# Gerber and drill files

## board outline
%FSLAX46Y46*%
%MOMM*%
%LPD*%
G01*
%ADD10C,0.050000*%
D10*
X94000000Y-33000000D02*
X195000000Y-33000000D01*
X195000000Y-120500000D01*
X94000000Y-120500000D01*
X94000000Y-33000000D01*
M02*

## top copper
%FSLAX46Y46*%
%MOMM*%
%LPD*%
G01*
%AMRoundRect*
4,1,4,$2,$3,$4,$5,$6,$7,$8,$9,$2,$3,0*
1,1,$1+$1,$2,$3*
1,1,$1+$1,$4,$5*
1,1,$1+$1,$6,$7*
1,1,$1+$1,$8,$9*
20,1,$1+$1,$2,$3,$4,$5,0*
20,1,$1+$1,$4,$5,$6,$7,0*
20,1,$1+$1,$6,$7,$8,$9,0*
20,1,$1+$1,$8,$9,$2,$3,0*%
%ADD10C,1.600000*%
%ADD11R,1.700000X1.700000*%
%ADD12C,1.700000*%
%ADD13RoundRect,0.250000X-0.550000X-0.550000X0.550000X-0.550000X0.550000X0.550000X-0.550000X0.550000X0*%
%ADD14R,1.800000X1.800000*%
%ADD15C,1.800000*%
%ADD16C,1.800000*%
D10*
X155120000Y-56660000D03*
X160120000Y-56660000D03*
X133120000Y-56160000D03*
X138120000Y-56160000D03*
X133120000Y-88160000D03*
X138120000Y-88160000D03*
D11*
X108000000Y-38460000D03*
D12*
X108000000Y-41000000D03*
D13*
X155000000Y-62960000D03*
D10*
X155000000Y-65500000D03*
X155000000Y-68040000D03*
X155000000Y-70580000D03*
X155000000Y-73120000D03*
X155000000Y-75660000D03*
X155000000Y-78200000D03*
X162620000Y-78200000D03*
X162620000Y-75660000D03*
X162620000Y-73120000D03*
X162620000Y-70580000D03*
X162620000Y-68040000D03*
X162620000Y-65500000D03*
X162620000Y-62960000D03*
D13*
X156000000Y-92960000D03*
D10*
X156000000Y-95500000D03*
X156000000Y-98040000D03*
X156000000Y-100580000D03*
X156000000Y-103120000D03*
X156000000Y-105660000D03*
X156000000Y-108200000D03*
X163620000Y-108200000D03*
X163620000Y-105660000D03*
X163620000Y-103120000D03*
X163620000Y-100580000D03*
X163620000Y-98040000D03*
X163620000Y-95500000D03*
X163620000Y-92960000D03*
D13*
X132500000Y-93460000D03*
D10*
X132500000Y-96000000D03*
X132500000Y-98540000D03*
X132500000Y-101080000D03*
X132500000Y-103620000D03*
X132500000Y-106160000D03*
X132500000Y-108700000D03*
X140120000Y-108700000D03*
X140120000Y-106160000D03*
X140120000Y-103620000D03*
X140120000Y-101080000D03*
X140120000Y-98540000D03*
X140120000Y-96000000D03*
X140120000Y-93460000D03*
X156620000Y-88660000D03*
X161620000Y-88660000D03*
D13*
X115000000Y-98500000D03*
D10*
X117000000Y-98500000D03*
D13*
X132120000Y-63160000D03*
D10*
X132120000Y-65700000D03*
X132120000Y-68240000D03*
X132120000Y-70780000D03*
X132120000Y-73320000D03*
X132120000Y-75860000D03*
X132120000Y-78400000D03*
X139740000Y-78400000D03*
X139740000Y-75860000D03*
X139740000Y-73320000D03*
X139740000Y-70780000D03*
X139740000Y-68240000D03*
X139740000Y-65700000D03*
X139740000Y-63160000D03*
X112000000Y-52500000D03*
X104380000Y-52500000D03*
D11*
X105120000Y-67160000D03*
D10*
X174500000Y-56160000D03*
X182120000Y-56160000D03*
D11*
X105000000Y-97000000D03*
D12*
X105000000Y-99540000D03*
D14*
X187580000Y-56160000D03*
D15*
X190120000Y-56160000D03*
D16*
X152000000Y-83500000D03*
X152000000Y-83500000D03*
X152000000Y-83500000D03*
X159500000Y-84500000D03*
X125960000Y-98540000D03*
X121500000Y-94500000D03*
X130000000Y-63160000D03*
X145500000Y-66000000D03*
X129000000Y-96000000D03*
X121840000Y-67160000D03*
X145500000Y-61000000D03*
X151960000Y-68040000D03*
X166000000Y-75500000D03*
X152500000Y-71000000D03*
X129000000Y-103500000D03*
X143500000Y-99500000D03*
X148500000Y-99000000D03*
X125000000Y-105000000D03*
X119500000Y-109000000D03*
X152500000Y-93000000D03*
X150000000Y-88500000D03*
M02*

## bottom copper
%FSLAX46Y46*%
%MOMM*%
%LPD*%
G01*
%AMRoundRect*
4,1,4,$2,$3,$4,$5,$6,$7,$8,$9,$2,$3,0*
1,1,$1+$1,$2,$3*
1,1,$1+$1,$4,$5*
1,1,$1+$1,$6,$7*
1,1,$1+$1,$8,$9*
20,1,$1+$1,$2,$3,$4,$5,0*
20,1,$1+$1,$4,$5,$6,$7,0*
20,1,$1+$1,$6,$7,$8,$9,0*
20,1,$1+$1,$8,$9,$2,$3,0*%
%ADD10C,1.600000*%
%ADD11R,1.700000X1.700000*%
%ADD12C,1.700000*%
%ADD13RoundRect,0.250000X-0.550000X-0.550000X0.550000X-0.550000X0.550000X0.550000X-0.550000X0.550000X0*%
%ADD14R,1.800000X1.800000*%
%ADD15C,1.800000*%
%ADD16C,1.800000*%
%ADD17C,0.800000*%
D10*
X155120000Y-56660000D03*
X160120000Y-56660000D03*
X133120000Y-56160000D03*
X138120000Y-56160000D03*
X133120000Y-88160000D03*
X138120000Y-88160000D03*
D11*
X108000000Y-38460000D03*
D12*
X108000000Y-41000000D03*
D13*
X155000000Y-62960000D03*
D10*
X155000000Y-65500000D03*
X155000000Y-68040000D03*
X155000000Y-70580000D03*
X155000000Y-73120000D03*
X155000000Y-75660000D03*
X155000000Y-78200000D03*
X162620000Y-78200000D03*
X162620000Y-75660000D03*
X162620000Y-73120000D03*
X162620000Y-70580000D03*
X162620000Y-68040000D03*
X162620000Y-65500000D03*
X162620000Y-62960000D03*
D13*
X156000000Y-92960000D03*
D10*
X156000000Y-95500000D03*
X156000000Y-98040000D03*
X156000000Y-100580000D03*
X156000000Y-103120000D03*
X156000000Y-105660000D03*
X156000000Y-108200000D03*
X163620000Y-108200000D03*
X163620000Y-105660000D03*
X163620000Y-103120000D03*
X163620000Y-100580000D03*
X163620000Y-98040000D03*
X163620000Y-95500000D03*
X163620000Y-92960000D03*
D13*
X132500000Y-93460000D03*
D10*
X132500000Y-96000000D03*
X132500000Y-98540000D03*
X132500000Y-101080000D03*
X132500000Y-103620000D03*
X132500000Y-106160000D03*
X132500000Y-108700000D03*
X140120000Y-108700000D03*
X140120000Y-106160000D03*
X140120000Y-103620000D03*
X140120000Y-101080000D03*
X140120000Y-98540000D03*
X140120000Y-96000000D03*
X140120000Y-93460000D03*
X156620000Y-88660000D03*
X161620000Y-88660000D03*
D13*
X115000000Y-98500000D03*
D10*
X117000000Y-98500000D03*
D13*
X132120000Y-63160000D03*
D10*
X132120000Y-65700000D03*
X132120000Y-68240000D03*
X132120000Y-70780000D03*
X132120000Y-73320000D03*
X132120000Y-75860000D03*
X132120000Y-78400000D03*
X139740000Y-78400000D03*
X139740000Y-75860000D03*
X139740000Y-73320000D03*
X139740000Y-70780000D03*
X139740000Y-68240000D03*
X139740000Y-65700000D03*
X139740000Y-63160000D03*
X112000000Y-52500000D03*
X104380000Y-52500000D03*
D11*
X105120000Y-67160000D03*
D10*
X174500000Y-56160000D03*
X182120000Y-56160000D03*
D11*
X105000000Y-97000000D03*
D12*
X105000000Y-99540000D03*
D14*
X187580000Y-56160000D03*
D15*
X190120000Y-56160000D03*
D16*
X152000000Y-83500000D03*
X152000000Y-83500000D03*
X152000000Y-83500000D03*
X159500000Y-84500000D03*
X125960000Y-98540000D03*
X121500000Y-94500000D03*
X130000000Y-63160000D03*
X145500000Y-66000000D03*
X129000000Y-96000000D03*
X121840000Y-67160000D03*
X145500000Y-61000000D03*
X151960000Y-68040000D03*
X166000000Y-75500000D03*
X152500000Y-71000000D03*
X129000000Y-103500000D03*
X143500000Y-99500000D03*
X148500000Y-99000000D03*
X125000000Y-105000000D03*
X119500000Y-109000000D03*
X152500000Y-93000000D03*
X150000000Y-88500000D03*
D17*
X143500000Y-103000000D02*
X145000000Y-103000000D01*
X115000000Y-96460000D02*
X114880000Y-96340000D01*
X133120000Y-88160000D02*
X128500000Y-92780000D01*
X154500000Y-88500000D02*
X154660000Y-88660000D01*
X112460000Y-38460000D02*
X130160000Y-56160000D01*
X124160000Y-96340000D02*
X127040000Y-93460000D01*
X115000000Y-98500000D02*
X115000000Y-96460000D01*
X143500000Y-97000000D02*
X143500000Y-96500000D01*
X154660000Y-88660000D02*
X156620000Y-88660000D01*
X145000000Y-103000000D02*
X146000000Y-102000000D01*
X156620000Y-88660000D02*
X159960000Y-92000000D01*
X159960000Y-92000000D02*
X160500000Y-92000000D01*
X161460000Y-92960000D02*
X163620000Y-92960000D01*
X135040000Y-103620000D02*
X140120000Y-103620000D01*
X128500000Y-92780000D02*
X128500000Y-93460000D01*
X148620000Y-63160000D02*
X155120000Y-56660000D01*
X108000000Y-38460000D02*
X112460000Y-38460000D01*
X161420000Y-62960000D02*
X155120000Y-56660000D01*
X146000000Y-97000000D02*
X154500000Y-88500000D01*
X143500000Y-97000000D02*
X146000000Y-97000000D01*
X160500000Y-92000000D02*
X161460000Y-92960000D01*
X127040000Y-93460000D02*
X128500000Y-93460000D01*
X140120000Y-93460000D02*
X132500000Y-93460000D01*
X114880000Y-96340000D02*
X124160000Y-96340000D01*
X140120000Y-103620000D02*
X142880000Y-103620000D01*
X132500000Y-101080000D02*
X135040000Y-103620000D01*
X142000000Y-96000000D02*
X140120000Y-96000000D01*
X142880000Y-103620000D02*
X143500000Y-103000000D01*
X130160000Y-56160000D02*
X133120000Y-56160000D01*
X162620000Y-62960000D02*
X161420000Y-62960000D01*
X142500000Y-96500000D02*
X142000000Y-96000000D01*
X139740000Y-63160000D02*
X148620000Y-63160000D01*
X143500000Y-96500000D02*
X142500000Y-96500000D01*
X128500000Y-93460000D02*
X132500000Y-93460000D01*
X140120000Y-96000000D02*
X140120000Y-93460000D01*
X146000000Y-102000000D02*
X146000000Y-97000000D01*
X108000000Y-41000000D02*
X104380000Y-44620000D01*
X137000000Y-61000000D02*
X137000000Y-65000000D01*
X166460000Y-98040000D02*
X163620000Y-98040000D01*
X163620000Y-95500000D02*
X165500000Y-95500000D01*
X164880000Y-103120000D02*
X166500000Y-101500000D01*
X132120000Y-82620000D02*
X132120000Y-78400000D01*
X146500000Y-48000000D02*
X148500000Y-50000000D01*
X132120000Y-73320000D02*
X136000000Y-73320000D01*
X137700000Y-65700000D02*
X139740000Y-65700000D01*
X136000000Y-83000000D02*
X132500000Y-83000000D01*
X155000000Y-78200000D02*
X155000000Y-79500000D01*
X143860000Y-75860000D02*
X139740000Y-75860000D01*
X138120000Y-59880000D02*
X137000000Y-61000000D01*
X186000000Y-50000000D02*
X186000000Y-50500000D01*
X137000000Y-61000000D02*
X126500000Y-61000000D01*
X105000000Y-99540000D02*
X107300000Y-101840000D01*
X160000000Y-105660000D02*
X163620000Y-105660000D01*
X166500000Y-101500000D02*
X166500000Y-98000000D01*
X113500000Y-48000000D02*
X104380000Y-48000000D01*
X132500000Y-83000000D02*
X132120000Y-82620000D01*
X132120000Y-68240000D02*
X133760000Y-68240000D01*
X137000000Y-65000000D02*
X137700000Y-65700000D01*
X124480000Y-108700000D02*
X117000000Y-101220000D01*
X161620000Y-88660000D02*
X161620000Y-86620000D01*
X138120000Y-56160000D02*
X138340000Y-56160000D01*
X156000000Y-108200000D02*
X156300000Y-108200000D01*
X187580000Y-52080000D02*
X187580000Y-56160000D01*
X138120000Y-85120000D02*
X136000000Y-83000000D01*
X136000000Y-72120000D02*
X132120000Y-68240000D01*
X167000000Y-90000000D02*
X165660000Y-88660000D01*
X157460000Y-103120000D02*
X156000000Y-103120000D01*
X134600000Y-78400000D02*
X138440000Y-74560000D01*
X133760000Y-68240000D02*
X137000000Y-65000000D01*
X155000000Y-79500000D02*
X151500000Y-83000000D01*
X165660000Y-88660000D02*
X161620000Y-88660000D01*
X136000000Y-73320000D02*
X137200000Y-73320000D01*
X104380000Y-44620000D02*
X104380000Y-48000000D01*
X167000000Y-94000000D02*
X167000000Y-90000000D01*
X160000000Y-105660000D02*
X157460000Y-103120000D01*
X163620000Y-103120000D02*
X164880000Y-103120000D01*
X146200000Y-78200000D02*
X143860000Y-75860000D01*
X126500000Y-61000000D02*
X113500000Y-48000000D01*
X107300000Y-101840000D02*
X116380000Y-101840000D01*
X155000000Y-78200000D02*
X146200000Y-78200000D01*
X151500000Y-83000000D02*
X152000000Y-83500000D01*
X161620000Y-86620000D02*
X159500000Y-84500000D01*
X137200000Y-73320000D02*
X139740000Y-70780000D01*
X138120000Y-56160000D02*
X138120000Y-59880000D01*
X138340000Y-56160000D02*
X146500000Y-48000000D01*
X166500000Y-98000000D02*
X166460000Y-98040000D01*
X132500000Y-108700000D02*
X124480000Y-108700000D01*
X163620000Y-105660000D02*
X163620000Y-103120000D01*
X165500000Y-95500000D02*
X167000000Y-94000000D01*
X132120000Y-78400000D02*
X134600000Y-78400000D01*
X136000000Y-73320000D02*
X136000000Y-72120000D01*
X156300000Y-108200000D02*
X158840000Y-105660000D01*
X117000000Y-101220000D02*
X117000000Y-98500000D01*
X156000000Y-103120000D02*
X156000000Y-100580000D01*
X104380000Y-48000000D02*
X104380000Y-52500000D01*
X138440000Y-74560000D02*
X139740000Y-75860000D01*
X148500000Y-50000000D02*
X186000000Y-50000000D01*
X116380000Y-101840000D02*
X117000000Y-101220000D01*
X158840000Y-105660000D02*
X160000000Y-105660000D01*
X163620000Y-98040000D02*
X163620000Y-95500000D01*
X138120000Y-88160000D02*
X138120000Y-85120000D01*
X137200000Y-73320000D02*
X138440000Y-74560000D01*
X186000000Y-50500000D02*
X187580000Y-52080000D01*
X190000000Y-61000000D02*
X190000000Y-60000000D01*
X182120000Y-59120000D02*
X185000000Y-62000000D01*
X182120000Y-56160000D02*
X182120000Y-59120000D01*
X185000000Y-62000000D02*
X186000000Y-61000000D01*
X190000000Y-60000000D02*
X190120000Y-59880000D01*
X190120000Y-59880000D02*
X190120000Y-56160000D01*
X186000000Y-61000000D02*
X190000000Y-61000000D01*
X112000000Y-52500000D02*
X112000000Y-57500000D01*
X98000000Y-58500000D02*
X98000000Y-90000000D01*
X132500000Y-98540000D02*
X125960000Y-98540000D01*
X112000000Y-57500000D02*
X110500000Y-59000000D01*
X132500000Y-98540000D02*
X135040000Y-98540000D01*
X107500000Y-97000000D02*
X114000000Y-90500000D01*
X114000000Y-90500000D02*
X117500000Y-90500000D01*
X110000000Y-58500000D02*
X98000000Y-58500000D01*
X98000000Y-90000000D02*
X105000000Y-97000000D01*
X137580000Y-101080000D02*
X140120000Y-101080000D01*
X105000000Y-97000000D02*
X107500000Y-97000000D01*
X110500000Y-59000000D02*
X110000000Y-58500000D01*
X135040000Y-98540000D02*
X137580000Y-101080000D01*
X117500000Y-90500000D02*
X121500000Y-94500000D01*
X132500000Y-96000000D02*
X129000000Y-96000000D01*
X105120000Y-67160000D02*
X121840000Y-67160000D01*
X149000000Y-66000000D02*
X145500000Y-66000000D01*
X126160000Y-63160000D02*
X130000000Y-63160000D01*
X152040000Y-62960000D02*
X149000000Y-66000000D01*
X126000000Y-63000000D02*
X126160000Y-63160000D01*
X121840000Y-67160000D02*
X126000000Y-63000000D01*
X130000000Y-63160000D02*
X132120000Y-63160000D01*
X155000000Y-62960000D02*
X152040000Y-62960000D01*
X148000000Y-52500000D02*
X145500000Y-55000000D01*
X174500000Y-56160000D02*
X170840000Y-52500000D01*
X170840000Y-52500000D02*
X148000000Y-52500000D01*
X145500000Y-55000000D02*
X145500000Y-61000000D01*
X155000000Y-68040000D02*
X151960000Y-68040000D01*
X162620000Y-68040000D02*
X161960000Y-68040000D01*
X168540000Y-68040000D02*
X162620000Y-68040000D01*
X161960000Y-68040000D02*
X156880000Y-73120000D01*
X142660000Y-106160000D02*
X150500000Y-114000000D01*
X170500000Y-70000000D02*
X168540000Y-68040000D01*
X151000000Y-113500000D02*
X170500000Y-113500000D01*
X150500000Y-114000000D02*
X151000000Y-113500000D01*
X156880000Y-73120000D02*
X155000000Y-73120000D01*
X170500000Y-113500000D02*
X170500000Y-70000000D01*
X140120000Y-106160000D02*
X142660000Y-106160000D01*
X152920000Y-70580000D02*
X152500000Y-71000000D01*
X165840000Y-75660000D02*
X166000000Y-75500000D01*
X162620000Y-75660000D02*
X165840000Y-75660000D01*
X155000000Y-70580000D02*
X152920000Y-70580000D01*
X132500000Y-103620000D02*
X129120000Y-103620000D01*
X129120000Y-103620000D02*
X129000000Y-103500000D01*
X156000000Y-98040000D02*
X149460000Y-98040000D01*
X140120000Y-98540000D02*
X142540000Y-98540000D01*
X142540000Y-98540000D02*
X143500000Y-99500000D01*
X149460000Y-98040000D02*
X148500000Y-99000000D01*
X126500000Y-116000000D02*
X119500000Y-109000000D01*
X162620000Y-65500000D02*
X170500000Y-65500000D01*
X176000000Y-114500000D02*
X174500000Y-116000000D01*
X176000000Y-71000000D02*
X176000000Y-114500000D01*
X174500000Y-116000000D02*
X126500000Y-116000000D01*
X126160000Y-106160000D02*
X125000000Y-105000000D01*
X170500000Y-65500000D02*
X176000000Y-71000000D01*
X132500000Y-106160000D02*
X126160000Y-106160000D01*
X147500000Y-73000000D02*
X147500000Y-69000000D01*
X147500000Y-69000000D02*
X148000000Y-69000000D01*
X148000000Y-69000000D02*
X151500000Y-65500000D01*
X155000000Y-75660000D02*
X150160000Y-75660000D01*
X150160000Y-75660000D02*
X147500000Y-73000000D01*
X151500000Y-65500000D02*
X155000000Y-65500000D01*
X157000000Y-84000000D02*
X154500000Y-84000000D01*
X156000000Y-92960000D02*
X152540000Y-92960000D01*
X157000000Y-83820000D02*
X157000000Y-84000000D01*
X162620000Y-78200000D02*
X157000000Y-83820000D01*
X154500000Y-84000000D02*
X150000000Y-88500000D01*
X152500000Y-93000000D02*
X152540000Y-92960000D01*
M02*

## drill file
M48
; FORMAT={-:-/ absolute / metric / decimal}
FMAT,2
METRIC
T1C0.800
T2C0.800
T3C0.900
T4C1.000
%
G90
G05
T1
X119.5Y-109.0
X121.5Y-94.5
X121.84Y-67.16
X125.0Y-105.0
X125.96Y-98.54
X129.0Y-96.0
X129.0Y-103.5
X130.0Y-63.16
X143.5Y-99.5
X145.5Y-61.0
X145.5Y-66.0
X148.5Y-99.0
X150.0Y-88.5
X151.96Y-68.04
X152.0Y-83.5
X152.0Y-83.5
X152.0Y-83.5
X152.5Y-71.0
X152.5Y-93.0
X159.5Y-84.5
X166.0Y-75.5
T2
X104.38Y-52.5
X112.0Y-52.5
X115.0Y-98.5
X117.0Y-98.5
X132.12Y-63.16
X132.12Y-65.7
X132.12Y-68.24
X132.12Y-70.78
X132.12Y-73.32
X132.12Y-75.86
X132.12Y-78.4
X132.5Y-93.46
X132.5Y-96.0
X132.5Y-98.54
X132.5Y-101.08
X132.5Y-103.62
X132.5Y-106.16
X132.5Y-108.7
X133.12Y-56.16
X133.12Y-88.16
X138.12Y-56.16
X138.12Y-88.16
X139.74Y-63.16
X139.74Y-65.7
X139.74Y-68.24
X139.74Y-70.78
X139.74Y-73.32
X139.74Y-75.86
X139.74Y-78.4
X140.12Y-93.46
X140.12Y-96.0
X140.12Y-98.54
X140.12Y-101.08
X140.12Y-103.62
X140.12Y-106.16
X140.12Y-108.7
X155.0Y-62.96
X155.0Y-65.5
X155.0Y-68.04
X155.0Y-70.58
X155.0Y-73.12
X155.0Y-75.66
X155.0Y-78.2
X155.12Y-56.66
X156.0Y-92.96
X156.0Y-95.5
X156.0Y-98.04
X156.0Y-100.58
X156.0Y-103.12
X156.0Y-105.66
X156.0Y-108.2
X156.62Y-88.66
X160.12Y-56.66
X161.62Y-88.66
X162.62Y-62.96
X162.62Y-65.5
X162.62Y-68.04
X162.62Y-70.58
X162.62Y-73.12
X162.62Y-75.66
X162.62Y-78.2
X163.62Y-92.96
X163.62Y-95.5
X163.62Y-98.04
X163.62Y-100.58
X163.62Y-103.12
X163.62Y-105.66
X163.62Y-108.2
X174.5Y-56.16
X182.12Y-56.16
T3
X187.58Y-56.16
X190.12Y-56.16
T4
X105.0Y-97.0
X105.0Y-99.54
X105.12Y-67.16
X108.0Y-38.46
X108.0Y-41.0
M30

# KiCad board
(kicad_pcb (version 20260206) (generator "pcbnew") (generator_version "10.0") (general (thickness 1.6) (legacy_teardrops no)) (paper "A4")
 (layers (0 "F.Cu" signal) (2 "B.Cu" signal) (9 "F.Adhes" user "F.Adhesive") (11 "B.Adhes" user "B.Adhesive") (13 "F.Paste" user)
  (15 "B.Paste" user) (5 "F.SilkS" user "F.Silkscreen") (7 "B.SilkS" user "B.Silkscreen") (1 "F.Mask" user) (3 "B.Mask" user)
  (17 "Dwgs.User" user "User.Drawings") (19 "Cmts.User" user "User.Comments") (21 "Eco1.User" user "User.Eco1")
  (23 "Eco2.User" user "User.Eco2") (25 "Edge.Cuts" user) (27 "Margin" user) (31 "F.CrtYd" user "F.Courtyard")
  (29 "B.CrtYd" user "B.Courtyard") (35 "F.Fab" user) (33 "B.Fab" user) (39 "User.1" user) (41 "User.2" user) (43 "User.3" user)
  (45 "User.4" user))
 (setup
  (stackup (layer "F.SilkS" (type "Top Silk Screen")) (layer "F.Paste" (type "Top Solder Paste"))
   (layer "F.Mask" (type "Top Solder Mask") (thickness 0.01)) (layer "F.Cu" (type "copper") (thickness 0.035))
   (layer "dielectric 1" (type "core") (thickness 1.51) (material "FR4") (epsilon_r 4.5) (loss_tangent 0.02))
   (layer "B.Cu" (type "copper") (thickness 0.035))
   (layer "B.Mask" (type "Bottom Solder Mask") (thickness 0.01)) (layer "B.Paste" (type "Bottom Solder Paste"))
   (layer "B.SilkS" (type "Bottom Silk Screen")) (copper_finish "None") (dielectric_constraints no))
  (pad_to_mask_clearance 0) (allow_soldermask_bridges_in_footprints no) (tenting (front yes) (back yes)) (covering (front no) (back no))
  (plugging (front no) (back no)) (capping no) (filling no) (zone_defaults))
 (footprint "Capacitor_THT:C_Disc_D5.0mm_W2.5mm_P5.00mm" (layer "F.Cu") (at 155.12 56.66)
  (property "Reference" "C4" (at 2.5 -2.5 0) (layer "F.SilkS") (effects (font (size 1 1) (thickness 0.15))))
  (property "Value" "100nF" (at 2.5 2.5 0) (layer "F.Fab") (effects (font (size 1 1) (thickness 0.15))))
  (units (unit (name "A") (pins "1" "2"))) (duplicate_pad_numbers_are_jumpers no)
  (pad "1" thru_hole circle (at 0 0) (size 1.6 1.6) (drill 0.8) (layers "*.Cu" "*.Mask") (remove_unused_layers no) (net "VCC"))
  (pad "2" thru_hole circle (at 5 0) (size 1.6 1.6) (drill 0.8) (layers "*.Cu" "*.Mask") (remove_unused_layers no) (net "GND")))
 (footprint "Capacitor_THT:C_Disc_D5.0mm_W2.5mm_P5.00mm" (layer "F.Cu") (at 133.12 56.16)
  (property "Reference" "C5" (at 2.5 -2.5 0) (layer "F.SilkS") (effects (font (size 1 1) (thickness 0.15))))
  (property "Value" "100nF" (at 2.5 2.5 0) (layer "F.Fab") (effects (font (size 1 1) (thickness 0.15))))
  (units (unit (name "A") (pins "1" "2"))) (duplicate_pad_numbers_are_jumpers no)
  (pad "1" thru_hole circle (at 0 0) (size 1.6 1.6) (drill 0.8) (layers "*.Cu" "*.Mask") (remove_unused_layers no) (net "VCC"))
  (pad "2" thru_hole circle (at 5 0) (size 1.6 1.6) (drill 0.8) (layers "*.Cu" "*.Mask") (remove_unused_layers no) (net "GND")))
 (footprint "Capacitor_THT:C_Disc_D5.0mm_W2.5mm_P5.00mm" (layer "F.Cu") (at 133.12 88.16)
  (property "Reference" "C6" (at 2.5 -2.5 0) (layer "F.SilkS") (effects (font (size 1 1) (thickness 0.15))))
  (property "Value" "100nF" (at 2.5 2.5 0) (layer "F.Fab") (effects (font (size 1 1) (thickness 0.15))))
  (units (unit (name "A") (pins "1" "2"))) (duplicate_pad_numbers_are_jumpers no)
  (pad "1" thru_hole circle (at 0 0) (size 1.6 1.6) (drill 0.8) (layers "*.Cu" "*.Mask") (remove_unused_layers no) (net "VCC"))
  (pad "2" thru_hole circle (at 5 0) (size 1.6 1.6) (drill 0.8) (layers "*.Cu" "*.Mask") (remove_unused_layers no) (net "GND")))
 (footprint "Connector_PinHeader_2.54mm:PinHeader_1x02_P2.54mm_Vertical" (layer "F.Cu") (at 108 38.46)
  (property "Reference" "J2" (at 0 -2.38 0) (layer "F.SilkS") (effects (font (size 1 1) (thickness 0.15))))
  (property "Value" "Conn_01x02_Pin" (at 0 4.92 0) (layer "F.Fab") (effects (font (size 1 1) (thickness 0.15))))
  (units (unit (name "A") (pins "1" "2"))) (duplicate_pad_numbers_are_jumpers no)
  (pad "1" thru_hole rect (at 0 0) (size 1.7 1.7) (drill 1) (layers "*.Cu" "*.Mask") (remove_unused_layers no) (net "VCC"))
  (pad "2" thru_hole circle (at 0 2.54) (size 1.7 1.7) (drill 1) (layers "*.Cu" "*.Mask") (remove_unused_layers no) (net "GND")))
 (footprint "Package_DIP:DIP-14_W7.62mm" (layer "F.Cu") (at 155 62.96)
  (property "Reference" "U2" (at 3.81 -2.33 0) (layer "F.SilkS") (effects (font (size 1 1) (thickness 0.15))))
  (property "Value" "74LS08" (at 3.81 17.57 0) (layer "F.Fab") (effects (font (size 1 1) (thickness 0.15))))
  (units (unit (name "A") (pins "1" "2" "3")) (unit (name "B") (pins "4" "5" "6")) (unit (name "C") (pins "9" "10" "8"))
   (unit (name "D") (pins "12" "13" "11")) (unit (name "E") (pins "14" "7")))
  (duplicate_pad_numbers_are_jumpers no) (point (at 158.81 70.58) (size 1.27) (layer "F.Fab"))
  (pad "1" thru_hole roundrect (at 0 0) (size 1.6 1.6) (drill 0.8) (layers "*.Cu" "*.Mask") (remove_unused_layers no)
   (roundrect_rratio 0.15625) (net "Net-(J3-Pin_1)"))
  (pad "2" thru_hole circle (at 0 2.54) (size 1.6 1.6) (drill 0.8) (layers "*.Cu" "*.Mask") (remove_unused_layers no) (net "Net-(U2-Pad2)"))
  (pad "3" thru_hole circle (at 0 5.08) (size 1.6 1.6) (drill 0.8) (layers "*.Cu" "*.Mask") (remove_unused_layers no) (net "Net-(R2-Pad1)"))
  (pad "4" thru_hole circle (at 0 7.62) (size 1.6 1.6) (drill 0.8) (layers "*.Cu" "*.Mask") (remove_unused_layers no) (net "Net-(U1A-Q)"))
  (pad "5" thru_hole circle (at 0 10.16) (size 1.6 1.6) (drill 0.8) (layers "*.Cu" "*.Mask") (remove_unused_layers no) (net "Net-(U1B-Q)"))
  (pad "6" thru_hole circle (at 0 12.7) (size 1.6 1.6) (drill 0.8) (layers "*.Cu" "*.Mask") (remove_unused_layers no) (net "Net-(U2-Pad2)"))
  (pad "7" thru_hole circle (at 0 15.24) (size 1.6 1.6) (drill 0.8) (layers "*.Cu" "*.Mask") (remove_unused_layers no) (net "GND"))
  (pad "8" thru_hole circle (at 7.62 15.24) (size 1.6 1.6) (drill 0.8) (layers "*.Cu" "*.Mask") (remove_unused_layers no)
   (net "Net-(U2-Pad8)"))
  (pad "9" thru_hole circle (at 7.62 12.7) (size 1.6 1.6) (drill 0.8) (layers "*.Cu" "*.Mask") (remove_unused_layers no) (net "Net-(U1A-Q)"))
  (pad "10" thru_hole circle (at 7.62 10.16) (size 1.6 1.6) (drill 0.8) (layers "*.Cu" "*.Mask") (remove_unused_layers no)
   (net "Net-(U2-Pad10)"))
  (pad "11" thru_hole circle (at 7.62 7.62) (size 1.6 1.6) (drill 0.8) (layers "*.Cu" "*.Mask") (remove_unused_layers no)
   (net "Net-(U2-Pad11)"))
  (pad "12" thru_hole circle (at 7.62 5.08) (size 1.6 1.6) (drill 0.8) (layers "*.Cu" "*.Mask") (remove_unused_layers no)
   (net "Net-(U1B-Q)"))
  (pad "13" thru_hole circle (at 7.62 2.54) (size 1.6 1.6) (drill 0.8) (layers "*.Cu" "*.Mask") (remove_unused_layers no)
   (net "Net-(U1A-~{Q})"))
  (pad "14" thru_hole circle (at 7.62 0) (size 1.6 1.6) (drill 0.8) (layers "*.Cu" "*.Mask") (remove_unused_layers no) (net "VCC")))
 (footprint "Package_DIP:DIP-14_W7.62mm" (layer "F.Cu") (at 156 92.96)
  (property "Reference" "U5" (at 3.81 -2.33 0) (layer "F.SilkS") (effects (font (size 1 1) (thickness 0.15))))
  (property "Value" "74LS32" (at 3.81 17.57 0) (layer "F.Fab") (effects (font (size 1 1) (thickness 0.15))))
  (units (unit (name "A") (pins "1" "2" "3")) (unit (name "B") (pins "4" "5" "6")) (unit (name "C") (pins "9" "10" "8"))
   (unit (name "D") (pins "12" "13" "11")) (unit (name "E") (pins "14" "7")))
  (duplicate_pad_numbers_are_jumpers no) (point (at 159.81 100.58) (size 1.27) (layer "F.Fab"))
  (pad "1" thru_hole roundrect (at 0 0) (size 1.6 1.6) (drill 0.8) (layers "*.Cu" "*.Mask") (remove_unused_layers no)
   (roundrect_rratio 0.15625) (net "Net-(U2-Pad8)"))
  (pad "2" thru_hole circle (at 0 2.54) (size 1.6 1.6) (drill 0.8) (layers "*.Cu" "*.Mask") (remove_unused_layers no) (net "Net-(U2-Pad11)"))
  (pad "3" thru_hole circle (at 0 5.08) (size 1.6 1.6) (drill 0.8) (layers "*.Cu" "*.Mask") (remove_unused_layers no) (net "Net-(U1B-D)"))
  (pad "4" thru_hole circle (at 0 7.62) (size 1.6 1.6) (drill 0.8) (layers "*.Cu" "*.Mask") (remove_unused_layers no) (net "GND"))
  (pad "5" thru_hole circle (at 0 10.16) (size 1.6 1.6) (drill 0.8) (layers "*.Cu" "*.Mask") (remove_unused_layers no) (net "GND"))
  (pad "6" thru_hole circle (at 0 12.7) (size 1.6 1.6) (drill 0.8) (layers "*.Cu" "*.Mask") (remove_unused_layers no)
   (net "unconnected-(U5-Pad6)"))
  (pad "7" thru_hole circle (at 0 15.24) (size 1.6 1.6) (drill 0.8) (layers "*.Cu" "*.Mask") (remove_unused_layers no) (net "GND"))
  (pad "8" thru_hole circle (at 7.62 15.24) (size 1.6 1.6) (drill 0.8) (layers "*.Cu" "*.Mask") (remove_unused_layers no)
   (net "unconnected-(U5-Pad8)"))
  (pad "9" thru_hole circle (at 7.62 12.7) (size 1.6 1.6) (drill 0.8) (layers "*.Cu" "*.Mask") (remove_unused_layers no) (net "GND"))
  (pad "10" thru_hole circle (at 7.62 10.16) (size 1.6 1.6) (drill 0.8) (layers "*.Cu" "*.Mask") (remove_unused_layers no) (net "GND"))
  (pad "11" thru_hole circle (at 7.62 7.62) (size 1.6 1.6) (drill 0.8) (layers "*.Cu" "*.Mask") (remove_unused_layers no)
   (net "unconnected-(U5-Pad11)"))
  (pad "12" thru_hole circle (at 7.62 5.08) (size 1.6 1.6) (drill 0.8) (layers "*.Cu" "*.Mask") (remove_unused_layers no) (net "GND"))
  (pad "13" thru_hole circle (at 7.62 2.54) (size 1.6 1.6) (drill 0.8) (layers "*.Cu" "*.Mask") (remove_unused_layers no) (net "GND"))
  (pad "14" thru_hole circle (at 7.62 0) (size 1.6 1.6) (drill 0.8) (layers "*.Cu" "*.Mask") (remove_unused_layers no) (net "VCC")))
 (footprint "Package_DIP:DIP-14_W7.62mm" (layer "F.Cu") (at 132.5 93.46)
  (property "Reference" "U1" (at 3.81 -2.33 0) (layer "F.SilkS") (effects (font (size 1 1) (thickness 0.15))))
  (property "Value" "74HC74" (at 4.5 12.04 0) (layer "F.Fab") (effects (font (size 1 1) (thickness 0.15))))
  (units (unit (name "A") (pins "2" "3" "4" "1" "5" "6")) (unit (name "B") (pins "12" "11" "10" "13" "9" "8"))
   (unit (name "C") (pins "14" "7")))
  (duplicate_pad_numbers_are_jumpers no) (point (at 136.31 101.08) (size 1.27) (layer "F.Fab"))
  (pad "1" thru_hole roundrect (at 0 0) (size 1.6 1.6) (drill 0.8) (layers "*.Cu" "*.Mask") (remove_unused_layers no)
   (roundrect_rratio 0.15625) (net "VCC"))
  (pad "2" thru_hole circle (at 0 2.54) (size 1.6 1.6) (drill 0.8) (layers "*.Cu" "*.Mask") (remove_unused_layers no) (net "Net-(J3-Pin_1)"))
  (pad "3" thru_hole circle (at 0 5.08) (size 1.6 1.6) (drill 0.8) (layers "*.Cu" "*.Mask") (remove_unused_layers no) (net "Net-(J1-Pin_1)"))
  (pad "4" thru_hole circle (at 0 7.62) (size 1.6 1.6) (drill 0.8) (layers "*.Cu" "*.Mask") (remove_unused_layers no) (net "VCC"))
  (pad "5" thru_hole circle (at 0 10.16) (size 1.6 1.6) (drill 0.8) (layers "*.Cu" "*.Mask") (remove_unused_layers no) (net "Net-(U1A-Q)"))
  (pad "6" thru_hole circle (at 0 12.7) (size 1.6 1.6) (drill 0.8) (layers "*.Cu" "*.Mask") (remove_unused_layers no) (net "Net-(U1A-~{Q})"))
  (pad "7" thru_hole circle (at 0 15.24) (size 1.6 1.6) (drill 0.8) (layers "*.Cu" "*.Mask") (remove_unused_layers no) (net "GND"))
  (pad "8" thru_hole circle (at 7.62 15.24) (size 1.6 1.6) (drill 0.8) (layers "*.Cu" "*.Mask") (remove_unused_layers no)
   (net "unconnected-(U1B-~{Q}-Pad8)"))
  (pad "9" thru_hole circle (at 7.62 12.7) (size 1.6 1.6) (drill 0.8) (layers "*.Cu" "*.Mask") (remove_unused_layers no) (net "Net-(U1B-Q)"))
  (pad "10" thru_hole circle (at 7.62 10.16) (size 1.6 1.6) (drill 0.8) (layers "*.Cu" "*.Mask") (remove_unused_layers no) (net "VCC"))
  (pad "11" thru_hole circle (at 7.62 7.62) (size 1.6 1.6) (drill 0.8) (layers "*.Cu" "*.Mask") (remove_unused_layers no)
   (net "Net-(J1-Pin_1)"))
  (pad "12" thru_hole circle (at 7.62 5.08) (size 1.6 1.6) (drill 0.8) (layers "*.Cu" "*.Mask") (remove_unused_layers no)
   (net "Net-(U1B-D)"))
  (pad "13" thru_hole circle (at 7.62 2.54) (size 1.6 1.6) (drill 0.8) (layers "*.Cu" "*.Mask") (remove_unused_layers no) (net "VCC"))
  (pad "14" thru_hole circle (at 7.62 0) (size 1.6 1.6) (drill 0.8) (layers "*.Cu" "*.Mask") (remove_unused_layers no) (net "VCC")))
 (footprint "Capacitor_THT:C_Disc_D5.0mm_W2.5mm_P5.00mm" (layer "F.Cu") (at 156.62 88.66)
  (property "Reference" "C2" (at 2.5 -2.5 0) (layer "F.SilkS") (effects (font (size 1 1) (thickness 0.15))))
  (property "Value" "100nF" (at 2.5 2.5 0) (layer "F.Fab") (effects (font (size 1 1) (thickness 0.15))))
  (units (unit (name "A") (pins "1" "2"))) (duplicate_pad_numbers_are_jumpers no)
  (pad "1" thru_hole circle (at 0 0) (size 1.6 1.6) (drill 0.8) (layers "*.Cu" "*.Mask") (remove_unused_layers no) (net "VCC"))
  (pad "2" thru_hole circle (at 5 0) (size 1.6 1.6) (drill 0.8) (layers "*.Cu" "*.Mask") (remove_unused_layers no) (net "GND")))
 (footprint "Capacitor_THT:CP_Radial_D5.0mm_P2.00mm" (layer "F.Cu") (at 115 98.5)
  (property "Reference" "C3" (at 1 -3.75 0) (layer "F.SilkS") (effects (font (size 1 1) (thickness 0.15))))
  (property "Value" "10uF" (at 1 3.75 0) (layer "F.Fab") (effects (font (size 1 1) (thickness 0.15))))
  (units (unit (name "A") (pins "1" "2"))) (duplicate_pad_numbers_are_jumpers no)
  (pad "1" thru_hole roundrect (at 0 0) (size 1.6 1.6) (drill 0.8) (layers "*.Cu" "*.Mask") (remove_unused_layers no)
   (roundrect_rratio 0.15625) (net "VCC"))
  (pad "2" thru_hole circle (at 2 0) (size 1.6 1.6) (drill 0.8) (layers "*.Cu" "*.Mask") (remove_unused_layers no) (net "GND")))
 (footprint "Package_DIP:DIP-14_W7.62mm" (layer "F.Cu") (at 132.12 63.16)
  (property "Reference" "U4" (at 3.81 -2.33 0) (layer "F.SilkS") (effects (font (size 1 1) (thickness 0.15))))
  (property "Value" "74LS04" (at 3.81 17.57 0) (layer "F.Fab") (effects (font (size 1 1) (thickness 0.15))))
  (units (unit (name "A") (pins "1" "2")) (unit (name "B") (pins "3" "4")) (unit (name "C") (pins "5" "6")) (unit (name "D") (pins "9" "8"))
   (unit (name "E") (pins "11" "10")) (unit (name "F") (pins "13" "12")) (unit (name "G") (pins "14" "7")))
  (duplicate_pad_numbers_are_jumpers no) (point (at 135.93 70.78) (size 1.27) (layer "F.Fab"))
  (pad "1" thru_hole roundrect (at 0 0) (size 1.6 1.6) (drill 0.8) (layers "*.Cu" "*.Mask") (remove_unused_layers no)
   (roundrect_rratio 0.15625) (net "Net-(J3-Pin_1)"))
  (pad "2" thru_hole circle (at 0 2.54) (size 1.6 1.6) (drill 0.8) (layers "*.Cu" "*.Mask") (remove_unused_layers no) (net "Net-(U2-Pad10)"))
  (pad "3" thru_hole circle (at 0 5.08) (size 1.6 1.6) (drill 0.8) (layers "*.Cu" "*.Mask") (remove_unused_layers no) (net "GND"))
  (pad "4" thru_hole circle (at 0 7.62) (size 1.6 1.6) (drill 0.8) (layers "*.Cu" "*.Mask") (remove_unused_layers no)
   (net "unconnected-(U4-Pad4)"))
  (pad "5" thru_hole circle (at 0 10.16) (size 1.6 1.6) (drill 0.8) (layers "*.Cu" "*.Mask") (remove_unused_layers no) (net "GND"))
  (pad "6" thru_hole circle (at 0 12.7) (size 1.6 1.6) (drill 0.8) (layers "*.Cu" "*.Mask") (remove_unused_layers no)
   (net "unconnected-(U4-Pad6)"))
  (pad "7" thru_hole circle (at 0 15.24) (size 1.6 1.6) (drill 0.8) (layers "*.Cu" "*.Mask") (remove_unused_layers no) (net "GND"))
  (pad "8" thru_hole circle (at 7.62 15.24) (size 1.6 1.6) (drill 0.8) (layers "*.Cu" "*.Mask") (remove_unused_layers no)
   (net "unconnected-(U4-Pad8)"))
  (pad "9" thru_hole circle (at 7.62 12.7) (size 1.6 1.6) (drill 0.8) (layers "*.Cu" "*.Mask") (remove_unused_layers no) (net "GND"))
  (pad "10" thru_hole circle (at 7.62 10.16) (size 1.6 1.6) (drill 0.8) (layers "*.Cu" "*.Mask") (remove_unused_layers no)
   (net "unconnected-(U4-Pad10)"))
  (pad "11" thru_hole circle (at 7.62 7.62) (size 1.6 1.6) (drill 0.8) (layers "*.Cu" "*.Mask") (remove_unused_layers no) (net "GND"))
  (pad "12" thru_hole circle (at 7.62 5.08) (size 1.6 1.6) (drill 0.8) (layers "*.Cu" "*.Mask") (remove_unused_layers no)
   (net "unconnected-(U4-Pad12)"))
  (pad "13" thru_hole circle (at 7.62 2.54) (size 1.6 1.6) (drill 0.8) (layers "*.Cu" "*.Mask") (remove_unused_layers no) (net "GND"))
  (pad "14" thru_hole circle (at 7.62 0) (size 1.6 1.6) (drill 0.8) (layers "*.Cu" "*.Mask") (remove_unused_layers no) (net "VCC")))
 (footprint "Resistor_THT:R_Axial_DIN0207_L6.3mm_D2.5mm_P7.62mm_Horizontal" (layer "F.Cu") (at 112 52.5 180)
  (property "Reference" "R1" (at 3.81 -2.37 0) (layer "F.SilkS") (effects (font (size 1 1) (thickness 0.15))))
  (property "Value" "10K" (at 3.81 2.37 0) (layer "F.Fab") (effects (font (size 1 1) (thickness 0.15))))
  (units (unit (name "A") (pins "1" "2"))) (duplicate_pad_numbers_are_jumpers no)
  (pad "1" thru_hole circle (at 0 0 180) (size 1.6 1.6) (drill 0.8) (layers "*.Cu" "*.Mask") (remove_unused_layers no)
   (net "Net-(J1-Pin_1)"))
  (pad "2" thru_hole circle (at 7.62 0 180) (size 1.6 1.6) (drill 0.8) (layers "*.Cu" "*.Mask") (remove_unused_layers no) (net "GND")))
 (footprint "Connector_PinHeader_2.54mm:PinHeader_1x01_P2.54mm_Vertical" (layer "F.Cu") (at 105.12 67.16)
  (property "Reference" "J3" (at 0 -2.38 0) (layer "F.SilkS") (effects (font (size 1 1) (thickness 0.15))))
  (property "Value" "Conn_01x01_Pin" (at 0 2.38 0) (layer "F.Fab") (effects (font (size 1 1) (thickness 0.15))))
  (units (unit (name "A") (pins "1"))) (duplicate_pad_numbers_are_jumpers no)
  (pad "1" thru_hole rect (at 0 0) (size 1.7 1.7) (drill 1) (layers "*.Cu" "*.Mask") (remove_unused_layers no) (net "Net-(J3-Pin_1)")))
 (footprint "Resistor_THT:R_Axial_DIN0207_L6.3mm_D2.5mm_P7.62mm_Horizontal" (layer "F.Cu") (at 174.5 56.16)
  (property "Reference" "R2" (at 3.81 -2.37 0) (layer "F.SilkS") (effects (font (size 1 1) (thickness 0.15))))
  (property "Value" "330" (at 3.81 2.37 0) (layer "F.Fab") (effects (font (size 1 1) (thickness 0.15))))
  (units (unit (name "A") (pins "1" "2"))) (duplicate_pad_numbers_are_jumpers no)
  (pad "1" thru_hole circle (at 0 0) (size 1.6 1.6) (drill 0.8) (layers "*.Cu" "*.Mask") (remove_unused_layers no) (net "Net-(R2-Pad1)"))
  (pad "2" thru_hole circle (at 7.62 0) (size 1.6 1.6) (drill 0.8) (layers "*.Cu" "*.Mask") (remove_unused_layers no) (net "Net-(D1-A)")))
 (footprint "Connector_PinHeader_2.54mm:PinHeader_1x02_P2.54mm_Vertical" (layer "F.Cu") (at 105 97)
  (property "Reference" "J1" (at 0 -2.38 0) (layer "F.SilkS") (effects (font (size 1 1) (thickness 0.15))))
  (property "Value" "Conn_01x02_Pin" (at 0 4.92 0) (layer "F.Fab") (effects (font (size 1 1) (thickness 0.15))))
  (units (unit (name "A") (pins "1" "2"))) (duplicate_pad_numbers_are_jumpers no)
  (pad "1" thru_hole rect (at 0 0) (size 1.7 1.7) (drill 1) (layers "*.Cu" "*.Mask") (remove_unused_layers no) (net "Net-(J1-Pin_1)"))
  (pad "2" thru_hole circle (at 0 2.54) (size 1.7 1.7) (drill 1) (layers "*.Cu" "*.Mask") (remove_unused_layers no) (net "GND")))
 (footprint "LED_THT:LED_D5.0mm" (layer "F.Cu") (at 187.58 56.16)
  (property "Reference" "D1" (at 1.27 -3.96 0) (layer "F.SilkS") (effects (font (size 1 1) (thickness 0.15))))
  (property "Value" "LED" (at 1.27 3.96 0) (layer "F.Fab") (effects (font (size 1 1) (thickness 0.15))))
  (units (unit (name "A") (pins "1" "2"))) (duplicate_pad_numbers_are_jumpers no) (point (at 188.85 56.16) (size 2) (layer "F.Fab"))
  (pad "1" thru_hole rect (at 0 0) (size 1.8 1.8) (drill 0.9) (layers "*.Cu" "*.Mask") (remove_unused_layers no) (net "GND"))
  (pad "2" thru_hole circle (at 2.54 0) (size 1.8 1.8) (drill 0.9) (layers "*.Cu" "*.Mask") (remove_unused_layers no) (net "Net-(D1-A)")))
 (gr_rect (start 94 33) (end 195 120.5) (stroke (width 0.05) (type solid)) (fill no) (layer "Edge.Cuts"))
 (segment (start 143.5 103) (end 145 103) (width 0.8) (layer "B.Cu") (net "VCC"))
 (segment (start 115 96.46) (end 114.88 96.34) (width 0.8) (layer "B.Cu") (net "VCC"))
 (segment (start 133.12 88.16) (end 128.5 92.78) (width 0.8) (layer "B.Cu") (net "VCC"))
 (segment (start 154.5 88.5) (end 154.66 88.66) (width 0.8) (layer "B.Cu") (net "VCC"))
 (segment (start 112.46 38.46) (end 130.16 56.16) (width 0.8) (layer "B.Cu") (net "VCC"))
 (segment (start 124.16 96.34) (end 127.04 93.46) (width 0.8) (layer "B.Cu") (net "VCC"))
 (segment (start 115 98.5) (end 115 96.46) (width 0.8) (layer "B.Cu") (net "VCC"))
 (segment (start 143.5 97) (end 143.5 96.5) (width 0.8) (layer "B.Cu") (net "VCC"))
 (segment (start 154.66 88.66) (end 156.62 88.66) (width 0.8) (layer "B.Cu") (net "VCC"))
 (segment (start 145 103) (end 146 102) (width 0.8) (layer "B.Cu") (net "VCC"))
 (segment (start 156.62 88.66) (end 159.96 92) (width 0.8) (layer "B.Cu") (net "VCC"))
 (segment (start 159.96 92) (end 160.5 92) (width 0.8) (layer "B.Cu") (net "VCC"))
 (segment (start 161.46 92.96) (end 163.62 92.96) (width 0.8) (layer "B.Cu") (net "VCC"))
 (segment (start 135.04 103.62) (end 140.12 103.62) (width 0.8) (layer "B.Cu") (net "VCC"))
 (segment (start 128.5 92.78) (end 128.5 93.46) (width 0.8) (layer "B.Cu") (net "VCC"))
 (segment (start 148.62 63.16) (end 155.12 56.66) (width 0.8) (layer "B.Cu") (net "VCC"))
 (segment (start 108 38.46) (end 112.46 38.46) (width 0.8) (layer "B.Cu") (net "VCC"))
 (segment (start 161.42 62.96) (end 155.12 56.66) (width 0.8) (layer "B.Cu") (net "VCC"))
 (segment (start 146 97) (end 154.5 88.5) (width 0.8) (layer "B.Cu") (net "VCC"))
 (segment (start 143.5 97) (end 146 97) (width 0.8) (layer "B.Cu") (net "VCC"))
 (segment (start 160.5 92) (end 161.46 92.96) (width 0.8) (layer "B.Cu") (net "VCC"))
 (segment (start 127.04 93.46) (end 128.5 93.46) (width 0.8) (layer "B.Cu") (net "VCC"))
 (segment (start 140.12 93.46) (end 132.5 93.46) (width 0.8) (layer "B.Cu") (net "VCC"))
 (segment (start 114.88 96.34) (end 124.16 96.34) (width 0.8) (layer "B.Cu") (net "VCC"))
 (segment (start 140.12 103.62) (end 142.88 103.62) (width 0.8) (layer "B.Cu") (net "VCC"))
 (segment (start 132.5 101.08) (end 135.04 103.62) (width 0.8) (layer "B.Cu") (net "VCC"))
 (segment (start 142 96) (end 140.12 96) (width 0.8) (layer "B.Cu") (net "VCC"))
 (segment (start 142.88 103.62) (end 143.5 103) (width 0.8) (layer "B.Cu") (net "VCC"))
 (segment (start 130.16 56.16) (end 133.12 56.16) (width 0.8) (layer "B.Cu") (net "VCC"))
 (segment (start 162.62 62.96) (end 161.42 62.96) (width 0.8) (layer "B.Cu") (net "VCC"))
 (segment (start 142.5 96.5) (end 142 96) (width 0.8) (layer "B.Cu") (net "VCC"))
 (segment (start 139.74 63.16) (end 148.62 63.16) (width 0.8) (layer "B.Cu") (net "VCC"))
 (segment (start 143.5 96.5) (end 142.5 96.5) (width 0.8) (layer "B.Cu") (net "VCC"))
 (segment (start 128.5 93.46) (end 132.5 93.46) (width 0.8) (layer "B.Cu") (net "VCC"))
 (segment (start 140.12 96) (end 140.12 93.46) (width 0.8) (layer "B.Cu") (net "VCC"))
 (segment (start 146 102) (end 146 97) (width 0.8) (layer "B.Cu") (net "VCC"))
 (via (at 152 83.5) (size 1.8) (drill 0.8) (layers "F.Cu" "B.Cu") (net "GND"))
 (via (at 152 83.5) (size 1.8) (drill 0.8) (layers "F.Cu" "B.Cu") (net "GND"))
 (via (at 152 83.5) (size 1.8) (drill 0.8) (layers "F.Cu" "B.Cu") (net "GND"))
 (via (at 159.5 84.5) (size 1.8) (drill 0.8) (layers "F.Cu" "B.Cu") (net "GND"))
 (segment (start 108 41) (end 104.38 44.62) (width 0.8) (layer "B.Cu") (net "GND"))
 (segment (start 137 61) (end 137 65) (width 0.8) (layer "B.Cu") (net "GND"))
 (segment (start 166.46 98.04) (end 163.62 98.04) (width 0.8) (layer "B.Cu") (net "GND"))
 (segment (start 163.62 95.5) (end 165.5 95.5) (width 0.8) (layer "B.Cu") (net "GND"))
 (segment (start 164.88 103.12) (end 166.5 101.5) (width 0.8) (layer "B.Cu") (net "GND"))
 (segment (start 132.12 82.62) (end 132.12 78.4) (width 0.8) (layer "B.Cu") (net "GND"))
 (segment (start 146.5 48) (end 148.5 50) (width 0.8) (layer "B.Cu") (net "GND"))
 (segment (start 132.12 73.32) (end 136 73.32) (width 0.8) (layer "B.Cu") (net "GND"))
 (segment (start 137.7 65.7) (end 139.74 65.7) (width 0.8) (layer "B.Cu") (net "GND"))
 (segment (start 136 83) (end 132.5 83) (width 0.8) (layer "B.Cu") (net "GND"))
 (segment (start 155 78.2) (end 155 79.5) (width 0.8) (layer "B.Cu") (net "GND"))
 (segment (start 143.86 75.86) (end 139.74 75.86) (width 0.8) (layer "B.Cu") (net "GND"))
 (segment (start 138.12 59.88) (end 137 61) (width 0.8) (layer "B.Cu") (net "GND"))
 (segment (start 186 50) (end 186 50.5) (width 0.8) (layer "B.Cu") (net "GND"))
 (segment (start 137 61) (end 126.5 61) (width 0.8) (layer "B.Cu") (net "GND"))
 (segment (start 105 99.54) (end 107.3 101.84) (width 0.8) (layer "B.Cu") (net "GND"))
 (segment (start 160 105.66) (end 163.62 105.66) (width 0.8) (layer "B.Cu") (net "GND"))
 (segment (start 166.5 101.5) (end 166.5 98) (width 0.8) (layer "B.Cu") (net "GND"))
 (segment (start 113.5 48) (end 104.38 48) (width 0.8) (layer "B.Cu") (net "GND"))
 (segment (start 132.5 83) (end 132.12 82.62) (width 0.8) (layer "B.Cu") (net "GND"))
 (segment (start 132.12 68.24) (end 133.76 68.24) (width 0.8) (layer "B.Cu") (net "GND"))
 (segment (start 137 65) (end 137.7 65.7) (width 0.8) (layer "B.Cu") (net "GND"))
 (segment (start 124.48 108.7) (end 117 101.22) (width 0.8) (layer "B.Cu") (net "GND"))
 (segment (start 161.62 88.66) (end 161.62 86.62) (width 0.8) (layer "B.Cu") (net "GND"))
 (segment (start 138.12 56.16) (end 138.34 56.16) (width 0.8) (layer "B.Cu") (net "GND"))
 (segment (start 156 108.2) (end 156.3 108.2) (width 0.8) (layer "B.Cu") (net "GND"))
 (segment (start 187.58 52.08) (end 187.58 56.16) (width 0.8) (layer "B.Cu") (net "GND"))
 (segment (start 138.12 85.12) (end 136 83) (width 0.8) (layer "B.Cu") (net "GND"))
 (segment (start 136 72.12) (end 132.12 68.24) (width 0.8) (layer "B.Cu") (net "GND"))
 (segment (start 167 90) (end 165.66 88.66) (width 0.8) (layer "B.Cu") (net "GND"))
 (segment (start 157.46 103.12) (end 156 103.12) (width 0.8) (layer "B.Cu") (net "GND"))
 (segment (start 134.6 78.4) (end 138.44 74.56) (width 0.8) (layer "B.Cu") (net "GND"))
 (segment (start 133.76 68.24) (end 137 65) (width 0.8) (layer "B.Cu") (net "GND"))
 (segment (start 155 79.5) (end 151.5 83) (width 0.8) (layer "B.Cu") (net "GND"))
 (segment (start 165.66 88.66) (end 161.62 88.66) (width 0.8) (layer "B.Cu") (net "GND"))
 (segment (start 136 73.32) (end 137.2 73.32) (width 0.8) (layer "B.Cu") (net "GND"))
 (segment (start 104.38 44.62) (end 104.38 48) (width 0.8) (layer "B.Cu") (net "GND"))
 (segment (start 167 94) (end 167 90) (width 0.8) (layer "B.Cu") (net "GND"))
 (segment (start 160 105.66) (end 157.46 103.12) (width 0.8) (layer "B.Cu") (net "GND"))
 (segment (start 163.62 103.12) (end 164.88 103.12) (width 0.8) (layer "B.Cu") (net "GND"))
 (segment (start 146.2 78.2) (end 143.86 75.86) (width 0.8) (layer "B.Cu") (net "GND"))
 (segment (start 126.5 61) (end 113.5 48) (width 0.8) (layer "B.Cu") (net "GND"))
 (segment (start 107.3 101.84) (end 116.38 101.84) (width 0.8) (layer "B.Cu") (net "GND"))
 (segment (start 155 78.2) (end 146.2 78.2) (width 0.8) (layer "B.Cu") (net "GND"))
 (segment (start 151.5 83) (end 152 83.5) (width 0.8) (layer "B.Cu") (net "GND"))
 (segment (start 161.62 86.62) (end 159.5 84.5) (width 0.8) (layer "B.Cu") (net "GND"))
 (segment (start 137.2 73.32) (end 139.74 70.78) (width 0.8) (layer "B.Cu") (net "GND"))
 (segment (start 138.12 56.16) (end 138.12 59.88) (width 0.8) (layer "B.Cu") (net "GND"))
 (segment (start 138.34 56.16) (end 146.5 48) (width 0.8) (layer "B.Cu") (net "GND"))
 (segment (start 166.5 98) (end 166.46 98.04) (width 0.8) (layer "B.Cu") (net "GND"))
 (segment (start 132.5 108.7) (end 124.48 108.7) (width 0.8) (layer "B.Cu") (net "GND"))
 (segment (start 163.62 105.66) (end 163.62 103.12) (width 0.8) (layer "B.Cu") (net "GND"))
 (segment (start 165.5 95.5) (end 167 94) (width 0.8) (layer "B.Cu") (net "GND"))
 (segment (start 132.12 78.4) (end 134.6 78.4) (width 0.8) (layer "B.Cu") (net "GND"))
 (segment (start 136 73.32) (end 136 72.12) (width 0.8) (layer "B.Cu") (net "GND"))
 (segment (start 156.3 108.2) (end 158.84 105.66) (width 0.8) (layer "B.Cu") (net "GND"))
 (segment (start 117 101.22) (end 117 98.5) (width 0.8) (layer "B.Cu") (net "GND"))
 (segment (start 156 103.12) (end 156 100.58) (width 0.8) (layer "B.Cu") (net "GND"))
 (segment (start 104.38 48) (end 104.38 52.5) (width 0.8) (layer "B.Cu") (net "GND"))
 (segment (start 138.44 74.56) (end 139.74 75.86) (width 0.8) (layer "B.Cu") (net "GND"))
 (segment (start 148.5 50) (end 186 50) (width 0.8) (layer "B.Cu") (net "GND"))
 (segment (start 116.38 101.84) (end 117 101.22) (width 0.8) (layer "B.Cu") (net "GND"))
 (segment (start 158.84 105.66) (end 160 105.66) (width 0.8) (layer "B.Cu") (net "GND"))
 (segment (start 163.62 98.04) (end 163.62 95.5) (width 0.8) (layer "B.Cu") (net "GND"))
 (segment (start 138.12 88.16) (end 138.12 85.12) (width 0.8) (layer "B.Cu") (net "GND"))
 (segment (start 137.2 73.32) (end 138.44 74.56) (width 0.8) (layer "B.Cu") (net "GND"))
 (segment (start 186 50.5) (end 187.58 52.08) (width 0.8) (layer "B.Cu") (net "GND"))
 (segment (start 190 61) (end 190 60) (width 0.8) (layer "B.Cu") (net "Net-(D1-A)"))
 (segment (start 182.12 59.12) (end 185 62) (width 0.8) (layer "B.Cu") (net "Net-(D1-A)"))
 (segment (start 182.12 56.16) (end 182.12 59.12) (width 0.8) (layer "B.Cu") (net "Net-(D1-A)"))
 (segment (start 185 62) (end 186 61) (width 0.8) (layer "B.Cu") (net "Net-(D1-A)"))
 (segment (start 190 60) (end 190.12 59.88) (width 0.8) (layer "B.Cu") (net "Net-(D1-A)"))
 (segment (start 190.12 59.88) (end 190.12 56.16) (width 0.8) (layer "B.Cu") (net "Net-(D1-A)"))
 (segment (start 186 61) (end 190 61) (width 0.8) (layer "B.Cu") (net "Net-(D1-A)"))
 (via (at 125.96 98.54) (size 1.8) (drill 0.8) (layers "F.Cu" "B.Cu") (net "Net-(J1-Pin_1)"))
 (via (at 121.5 94.5) (size 1.8) (drill 0.8) (layers "F.Cu" "B.Cu") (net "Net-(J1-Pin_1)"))
 (segment (start 112 52.5) (end 112 57.5) (width 0.8) (layer "B.Cu") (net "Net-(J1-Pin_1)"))
 (segment (start 98 58.5) (end 98 90) (width 0.8) (layer "B.Cu") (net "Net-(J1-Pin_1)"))
 (segment (start 132.5 98.54) (end 125.96 98.54) (width 0.8) (layer "B.Cu") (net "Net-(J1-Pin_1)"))
 (segment (start 112 57.5) (end 110.5 59) (width 0.8) (layer "B.Cu") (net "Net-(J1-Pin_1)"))
 (segment (start 132.5 98.54) (end 135.04 98.54) (width 0.8) (layer "B.Cu") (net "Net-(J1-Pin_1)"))
 (segment (start 107.5 97) (end 114 90.5) (width 0.8) (layer "B.Cu") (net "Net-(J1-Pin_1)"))
 (segment (start 114 90.5) (end 117.5 90.5) (width 0.8) (layer "B.Cu") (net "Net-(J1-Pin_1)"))
 (segment (start 110 58.5) (end 98 58.5) (width 0.8) (layer "B.Cu") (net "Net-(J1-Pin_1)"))
 (segment (start 98 90) (end 105 97) (width 0.8) (layer "B.Cu") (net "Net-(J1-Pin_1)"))
 (segment (start 137.58 101.08) (end 140.12 101.08) (width 0.8) (layer "B.Cu") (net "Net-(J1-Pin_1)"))
 (segment (start 105 97) (end 107.5 97) (width 0.8) (layer "B.Cu") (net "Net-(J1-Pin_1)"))
 (segment (start 110.5 59) (end 110 58.5) (width 0.8) (layer "B.Cu") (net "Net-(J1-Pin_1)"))
 (segment (start 135.04 98.54) (end 137.58 101.08) (width 0.8) (layer "B.Cu") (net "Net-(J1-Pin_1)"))
 (segment (start 117.5 90.5) (end 121.5 94.5) (width 0.8) (layer "B.Cu") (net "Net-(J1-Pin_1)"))
 (via (at 130 63.16) (size 1.8) (drill 0.8) (layers "F.Cu" "B.Cu") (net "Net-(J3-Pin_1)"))
 (via (at 145.5 66) (size 1.8) (drill 0.8) (layers "F.Cu" "B.Cu") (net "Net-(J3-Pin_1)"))
 (via (at 129 96) (size 1.8) (drill 0.8) (layers "F.Cu" "B.Cu") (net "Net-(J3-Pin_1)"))
 (via (at 121.84 67.16) (size 1.8) (drill 0.8) (layers "F.Cu" "B.Cu") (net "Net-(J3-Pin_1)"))
 (segment (start 132.5 96) (end 129 96) (width 0.8) (layer "B.Cu") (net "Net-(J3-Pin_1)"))
 (segment (start 105.12 67.16) (end 121.84 67.16) (width 0.8) (layer "B.Cu") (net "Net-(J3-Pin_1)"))
 (segment (start 149 66) (end 145.5 66) (width 0.8) (layer "B.Cu") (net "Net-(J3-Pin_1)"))
 (segment (start 126.16 63.16) (end 130 63.16) (width 0.8) (layer "B.Cu") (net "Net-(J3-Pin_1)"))
 (segment (start 152.04 62.96) (end 149 66) (width 0.8) (layer "B.Cu") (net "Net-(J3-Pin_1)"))
 (segment (start 126 63) (end 126.16 63.16) (width 0.8) (layer "B.Cu") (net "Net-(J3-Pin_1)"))
 (segment (start 121.84 67.16) (end 126 63) (width 0.8) (layer "B.Cu") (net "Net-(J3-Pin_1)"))
 (segment (start 130 63.16) (end 132.12 63.16) (width 0.8) (layer "B.Cu") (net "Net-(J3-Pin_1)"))
 (segment (start 155 62.96) (end 152.04 62.96) (width 0.8) (layer "B.Cu") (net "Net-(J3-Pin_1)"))
 (via (at 145.5 61) (size 1.8) (drill 0.8) (layers "F.Cu" "B.Cu") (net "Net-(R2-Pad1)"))
 (via (at 151.96 68.04) (size 1.8) (drill 0.8) (layers "F.Cu" "B.Cu") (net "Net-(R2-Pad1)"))
 (segment (start 148 52.5) (end 145.5 55) (width 0.8) (layer "B.Cu") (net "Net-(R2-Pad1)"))
 (segment (start 174.5 56.16) (end 170.84 52.5) (width 0.8) (layer "B.Cu") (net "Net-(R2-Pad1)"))
 (segment (start 170.84 52.5) (end 148 52.5) (width 0.8) (layer "B.Cu") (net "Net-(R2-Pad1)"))
 (segment (start 145.5 55) (end 145.5 61) (width 0.8) (layer "B.Cu") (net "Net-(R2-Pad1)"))
 (segment (start 155 68.04) (end 151.96 68.04) (width 0.8) (layer "B.Cu") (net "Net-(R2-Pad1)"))
 (segment (start 162.62 68.04) (end 161.96 68.04) (width 0.8) (layer "B.Cu") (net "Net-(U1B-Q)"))
 (segment (start 168.54 68.04) (end 162.62 68.04) (width 0.8) (layer "B.Cu") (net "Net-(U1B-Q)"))
 (segment (start 161.96 68.04) (end 156.88 73.12) (width 0.8) (layer "B.Cu") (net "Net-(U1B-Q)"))
 (segment (start 142.66 106.16) (end 150.5 114) (width 0.8) (layer "B.Cu") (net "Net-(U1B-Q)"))
 (segment (start 170.5 70) (end 168.54 68.04) (width 0.8) (layer "B.Cu") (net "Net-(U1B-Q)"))
 (segment (start 151 113.5) (end 170.5 113.5) (width 0.8) (layer "B.Cu") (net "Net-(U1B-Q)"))
 (segment (start 150.5 114) (end 151 113.5) (width 0.8) (layer "B.Cu") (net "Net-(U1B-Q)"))
 (segment (start 156.88 73.12) (end 155 73.12) (width 0.8) (layer "B.Cu") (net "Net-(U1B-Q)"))
 (segment (start 170.5 113.5) (end 170.5 70) (width 0.8) (layer "B.Cu") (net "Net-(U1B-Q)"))
 (segment (start 140.12 106.16) (end 142.66 106.16) (width 0.8) (layer "B.Cu") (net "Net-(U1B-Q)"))
 (via (at 166 75.5) (size 1.8) (drill 0.8) (layers "F.Cu" "B.Cu") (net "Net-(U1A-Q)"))
 (via (at 152.5 71) (size 1.8) (drill 0.8) (layers "F.Cu" "B.Cu") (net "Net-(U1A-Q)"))
 (via (at 129 103.5) (size 1.8) (drill 0.8) (layers "F.Cu" "B.Cu") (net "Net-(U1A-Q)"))
 (segment (start 152.92 70.58) (end 152.5 71) (width 0.8) (layer "B.Cu") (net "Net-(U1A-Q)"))
 (segment (start 165.84 75.66) (end 166 75.5) (width 0.8) (layer "B.Cu") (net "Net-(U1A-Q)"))
 (segment (start 162.62 75.66) (end 165.84 75.66) (width 0.8) (layer "B.Cu") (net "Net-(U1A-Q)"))
 (segment (start 155 70.58) (end 152.92 70.58) (width 0.8) (layer "B.Cu") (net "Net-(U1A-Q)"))
 (segment (start 132.5 103.62) (end 129.12 103.62) (width 0.8) (layer "B.Cu") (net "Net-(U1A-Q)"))
 (segment (start 129.12 103.62) (end 129 103.5) (width 0.8) (layer "B.Cu") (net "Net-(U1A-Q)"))
 (via (at 143.5 99.5) (size 1.8) (drill 0.8) (layers "F.Cu" "B.Cu") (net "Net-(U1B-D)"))
 (via (at 148.5 99) (size 1.8) (drill 0.8) (layers "F.Cu" "B.Cu") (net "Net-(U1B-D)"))
 (segment (start 156 98.04) (end 149.46 98.04) (width 0.8) (layer "B.Cu") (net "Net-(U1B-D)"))
 (segment (start 140.12 98.54) (end 142.54 98.54) (width 0.8) (layer "B.Cu") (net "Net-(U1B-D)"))
 (segment (start 142.54 98.54) (end 143.5 99.5) (width 0.8) (layer "B.Cu") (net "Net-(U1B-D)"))
 (segment (start 149.46 98.04) (end 148.5 99) (width 0.8) (layer "B.Cu") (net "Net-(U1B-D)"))
 (via (at 125 105) (size 1.8) (drill 0.8) (layers "F.Cu" "B.Cu") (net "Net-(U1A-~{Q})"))
 (via (at 119.5 109) (size 1.8) (drill 0.8) (layers "F.Cu" "B.Cu") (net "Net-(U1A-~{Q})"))
 (segment (start 126.5 116) (end 119.5 109) (width 0.8) (layer "B.Cu") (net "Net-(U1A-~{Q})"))
 (segment (start 162.62 65.5) (end 170.5 65.5) (width 0.8) (layer "B.Cu") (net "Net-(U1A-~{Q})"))
 (segment (start 176 114.5) (end 174.5 116) (width 0.8) (layer "B.Cu") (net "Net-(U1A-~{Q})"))
 (segment (start 176 71) (end 176 114.5) (width 0.8) (layer "B.Cu") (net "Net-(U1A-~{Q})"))
 (segment (start 174.5 116) (end 126.5 116) (width 0.8) (layer "B.Cu") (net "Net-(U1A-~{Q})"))
 (segment (start 126.16 106.16) (end 125 105) (width 0.8) (layer "B.Cu") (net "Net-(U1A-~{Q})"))
 (segment (start 170.5 65.5) (end 176 71) (width 0.8) (layer "B.Cu") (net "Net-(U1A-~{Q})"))
 (segment (start 132.5 106.16) (end 126.16 106.16) (width 0.8) (layer "B.Cu") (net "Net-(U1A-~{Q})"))
 (segment (start 147.5 73) (end 147.5 69) (width 0.8) (layer "B.Cu") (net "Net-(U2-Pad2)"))
 (segment (start 147.5 69) (end 148 69) (width 0.8) (layer "B.Cu") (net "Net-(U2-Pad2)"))
 (segment (start 148 69) (end 151.5 65.5) (width 0.8) (layer "B.Cu") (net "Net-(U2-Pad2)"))
 (segment (start 155 75.66) (end 150.16 75.66) (width 0.8) (layer "B.Cu") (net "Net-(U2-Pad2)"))
 (segment (start 150.16 75.66) (end 147.5 73) (width 0.8) (layer "B.Cu") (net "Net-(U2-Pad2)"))
 (segment (start 151.5 65.5) (end 155 65.5) (width 0.8) (layer "B.Cu") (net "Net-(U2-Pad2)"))
 (via (at 152.5 93) (size 1.8) (drill 0.8) (layers "F.Cu" "B.Cu") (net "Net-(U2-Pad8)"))
 (via (at 150 88.5) (size 1.8) (drill 0.8) (layers "F.Cu" "B.Cu") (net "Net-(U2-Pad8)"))
 (segment (start 157 84) (end 154.5 84) (width 0.8) (layer "B.Cu") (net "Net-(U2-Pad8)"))
 (segment (start 156 92.96) (end 152.54 92.96) (width 0.8) (layer "B.Cu") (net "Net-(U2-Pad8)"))
 (segment (start 157 83.82) (end 157 84) (width 0.8) (layer "B.Cu") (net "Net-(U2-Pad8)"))
 (segment (start 162.62 78.2) (end 157 83.82) (width 0.8) (layer "B.Cu") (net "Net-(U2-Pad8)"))
 (segment (start 154.5 84) (end 150 88.5) (width 0.8) (layer "B.Cu") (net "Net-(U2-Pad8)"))
 (segment (start 152.5 93) (end 152.54 92.96) (width 0.8) (layer "B.Cu") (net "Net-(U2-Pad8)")))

